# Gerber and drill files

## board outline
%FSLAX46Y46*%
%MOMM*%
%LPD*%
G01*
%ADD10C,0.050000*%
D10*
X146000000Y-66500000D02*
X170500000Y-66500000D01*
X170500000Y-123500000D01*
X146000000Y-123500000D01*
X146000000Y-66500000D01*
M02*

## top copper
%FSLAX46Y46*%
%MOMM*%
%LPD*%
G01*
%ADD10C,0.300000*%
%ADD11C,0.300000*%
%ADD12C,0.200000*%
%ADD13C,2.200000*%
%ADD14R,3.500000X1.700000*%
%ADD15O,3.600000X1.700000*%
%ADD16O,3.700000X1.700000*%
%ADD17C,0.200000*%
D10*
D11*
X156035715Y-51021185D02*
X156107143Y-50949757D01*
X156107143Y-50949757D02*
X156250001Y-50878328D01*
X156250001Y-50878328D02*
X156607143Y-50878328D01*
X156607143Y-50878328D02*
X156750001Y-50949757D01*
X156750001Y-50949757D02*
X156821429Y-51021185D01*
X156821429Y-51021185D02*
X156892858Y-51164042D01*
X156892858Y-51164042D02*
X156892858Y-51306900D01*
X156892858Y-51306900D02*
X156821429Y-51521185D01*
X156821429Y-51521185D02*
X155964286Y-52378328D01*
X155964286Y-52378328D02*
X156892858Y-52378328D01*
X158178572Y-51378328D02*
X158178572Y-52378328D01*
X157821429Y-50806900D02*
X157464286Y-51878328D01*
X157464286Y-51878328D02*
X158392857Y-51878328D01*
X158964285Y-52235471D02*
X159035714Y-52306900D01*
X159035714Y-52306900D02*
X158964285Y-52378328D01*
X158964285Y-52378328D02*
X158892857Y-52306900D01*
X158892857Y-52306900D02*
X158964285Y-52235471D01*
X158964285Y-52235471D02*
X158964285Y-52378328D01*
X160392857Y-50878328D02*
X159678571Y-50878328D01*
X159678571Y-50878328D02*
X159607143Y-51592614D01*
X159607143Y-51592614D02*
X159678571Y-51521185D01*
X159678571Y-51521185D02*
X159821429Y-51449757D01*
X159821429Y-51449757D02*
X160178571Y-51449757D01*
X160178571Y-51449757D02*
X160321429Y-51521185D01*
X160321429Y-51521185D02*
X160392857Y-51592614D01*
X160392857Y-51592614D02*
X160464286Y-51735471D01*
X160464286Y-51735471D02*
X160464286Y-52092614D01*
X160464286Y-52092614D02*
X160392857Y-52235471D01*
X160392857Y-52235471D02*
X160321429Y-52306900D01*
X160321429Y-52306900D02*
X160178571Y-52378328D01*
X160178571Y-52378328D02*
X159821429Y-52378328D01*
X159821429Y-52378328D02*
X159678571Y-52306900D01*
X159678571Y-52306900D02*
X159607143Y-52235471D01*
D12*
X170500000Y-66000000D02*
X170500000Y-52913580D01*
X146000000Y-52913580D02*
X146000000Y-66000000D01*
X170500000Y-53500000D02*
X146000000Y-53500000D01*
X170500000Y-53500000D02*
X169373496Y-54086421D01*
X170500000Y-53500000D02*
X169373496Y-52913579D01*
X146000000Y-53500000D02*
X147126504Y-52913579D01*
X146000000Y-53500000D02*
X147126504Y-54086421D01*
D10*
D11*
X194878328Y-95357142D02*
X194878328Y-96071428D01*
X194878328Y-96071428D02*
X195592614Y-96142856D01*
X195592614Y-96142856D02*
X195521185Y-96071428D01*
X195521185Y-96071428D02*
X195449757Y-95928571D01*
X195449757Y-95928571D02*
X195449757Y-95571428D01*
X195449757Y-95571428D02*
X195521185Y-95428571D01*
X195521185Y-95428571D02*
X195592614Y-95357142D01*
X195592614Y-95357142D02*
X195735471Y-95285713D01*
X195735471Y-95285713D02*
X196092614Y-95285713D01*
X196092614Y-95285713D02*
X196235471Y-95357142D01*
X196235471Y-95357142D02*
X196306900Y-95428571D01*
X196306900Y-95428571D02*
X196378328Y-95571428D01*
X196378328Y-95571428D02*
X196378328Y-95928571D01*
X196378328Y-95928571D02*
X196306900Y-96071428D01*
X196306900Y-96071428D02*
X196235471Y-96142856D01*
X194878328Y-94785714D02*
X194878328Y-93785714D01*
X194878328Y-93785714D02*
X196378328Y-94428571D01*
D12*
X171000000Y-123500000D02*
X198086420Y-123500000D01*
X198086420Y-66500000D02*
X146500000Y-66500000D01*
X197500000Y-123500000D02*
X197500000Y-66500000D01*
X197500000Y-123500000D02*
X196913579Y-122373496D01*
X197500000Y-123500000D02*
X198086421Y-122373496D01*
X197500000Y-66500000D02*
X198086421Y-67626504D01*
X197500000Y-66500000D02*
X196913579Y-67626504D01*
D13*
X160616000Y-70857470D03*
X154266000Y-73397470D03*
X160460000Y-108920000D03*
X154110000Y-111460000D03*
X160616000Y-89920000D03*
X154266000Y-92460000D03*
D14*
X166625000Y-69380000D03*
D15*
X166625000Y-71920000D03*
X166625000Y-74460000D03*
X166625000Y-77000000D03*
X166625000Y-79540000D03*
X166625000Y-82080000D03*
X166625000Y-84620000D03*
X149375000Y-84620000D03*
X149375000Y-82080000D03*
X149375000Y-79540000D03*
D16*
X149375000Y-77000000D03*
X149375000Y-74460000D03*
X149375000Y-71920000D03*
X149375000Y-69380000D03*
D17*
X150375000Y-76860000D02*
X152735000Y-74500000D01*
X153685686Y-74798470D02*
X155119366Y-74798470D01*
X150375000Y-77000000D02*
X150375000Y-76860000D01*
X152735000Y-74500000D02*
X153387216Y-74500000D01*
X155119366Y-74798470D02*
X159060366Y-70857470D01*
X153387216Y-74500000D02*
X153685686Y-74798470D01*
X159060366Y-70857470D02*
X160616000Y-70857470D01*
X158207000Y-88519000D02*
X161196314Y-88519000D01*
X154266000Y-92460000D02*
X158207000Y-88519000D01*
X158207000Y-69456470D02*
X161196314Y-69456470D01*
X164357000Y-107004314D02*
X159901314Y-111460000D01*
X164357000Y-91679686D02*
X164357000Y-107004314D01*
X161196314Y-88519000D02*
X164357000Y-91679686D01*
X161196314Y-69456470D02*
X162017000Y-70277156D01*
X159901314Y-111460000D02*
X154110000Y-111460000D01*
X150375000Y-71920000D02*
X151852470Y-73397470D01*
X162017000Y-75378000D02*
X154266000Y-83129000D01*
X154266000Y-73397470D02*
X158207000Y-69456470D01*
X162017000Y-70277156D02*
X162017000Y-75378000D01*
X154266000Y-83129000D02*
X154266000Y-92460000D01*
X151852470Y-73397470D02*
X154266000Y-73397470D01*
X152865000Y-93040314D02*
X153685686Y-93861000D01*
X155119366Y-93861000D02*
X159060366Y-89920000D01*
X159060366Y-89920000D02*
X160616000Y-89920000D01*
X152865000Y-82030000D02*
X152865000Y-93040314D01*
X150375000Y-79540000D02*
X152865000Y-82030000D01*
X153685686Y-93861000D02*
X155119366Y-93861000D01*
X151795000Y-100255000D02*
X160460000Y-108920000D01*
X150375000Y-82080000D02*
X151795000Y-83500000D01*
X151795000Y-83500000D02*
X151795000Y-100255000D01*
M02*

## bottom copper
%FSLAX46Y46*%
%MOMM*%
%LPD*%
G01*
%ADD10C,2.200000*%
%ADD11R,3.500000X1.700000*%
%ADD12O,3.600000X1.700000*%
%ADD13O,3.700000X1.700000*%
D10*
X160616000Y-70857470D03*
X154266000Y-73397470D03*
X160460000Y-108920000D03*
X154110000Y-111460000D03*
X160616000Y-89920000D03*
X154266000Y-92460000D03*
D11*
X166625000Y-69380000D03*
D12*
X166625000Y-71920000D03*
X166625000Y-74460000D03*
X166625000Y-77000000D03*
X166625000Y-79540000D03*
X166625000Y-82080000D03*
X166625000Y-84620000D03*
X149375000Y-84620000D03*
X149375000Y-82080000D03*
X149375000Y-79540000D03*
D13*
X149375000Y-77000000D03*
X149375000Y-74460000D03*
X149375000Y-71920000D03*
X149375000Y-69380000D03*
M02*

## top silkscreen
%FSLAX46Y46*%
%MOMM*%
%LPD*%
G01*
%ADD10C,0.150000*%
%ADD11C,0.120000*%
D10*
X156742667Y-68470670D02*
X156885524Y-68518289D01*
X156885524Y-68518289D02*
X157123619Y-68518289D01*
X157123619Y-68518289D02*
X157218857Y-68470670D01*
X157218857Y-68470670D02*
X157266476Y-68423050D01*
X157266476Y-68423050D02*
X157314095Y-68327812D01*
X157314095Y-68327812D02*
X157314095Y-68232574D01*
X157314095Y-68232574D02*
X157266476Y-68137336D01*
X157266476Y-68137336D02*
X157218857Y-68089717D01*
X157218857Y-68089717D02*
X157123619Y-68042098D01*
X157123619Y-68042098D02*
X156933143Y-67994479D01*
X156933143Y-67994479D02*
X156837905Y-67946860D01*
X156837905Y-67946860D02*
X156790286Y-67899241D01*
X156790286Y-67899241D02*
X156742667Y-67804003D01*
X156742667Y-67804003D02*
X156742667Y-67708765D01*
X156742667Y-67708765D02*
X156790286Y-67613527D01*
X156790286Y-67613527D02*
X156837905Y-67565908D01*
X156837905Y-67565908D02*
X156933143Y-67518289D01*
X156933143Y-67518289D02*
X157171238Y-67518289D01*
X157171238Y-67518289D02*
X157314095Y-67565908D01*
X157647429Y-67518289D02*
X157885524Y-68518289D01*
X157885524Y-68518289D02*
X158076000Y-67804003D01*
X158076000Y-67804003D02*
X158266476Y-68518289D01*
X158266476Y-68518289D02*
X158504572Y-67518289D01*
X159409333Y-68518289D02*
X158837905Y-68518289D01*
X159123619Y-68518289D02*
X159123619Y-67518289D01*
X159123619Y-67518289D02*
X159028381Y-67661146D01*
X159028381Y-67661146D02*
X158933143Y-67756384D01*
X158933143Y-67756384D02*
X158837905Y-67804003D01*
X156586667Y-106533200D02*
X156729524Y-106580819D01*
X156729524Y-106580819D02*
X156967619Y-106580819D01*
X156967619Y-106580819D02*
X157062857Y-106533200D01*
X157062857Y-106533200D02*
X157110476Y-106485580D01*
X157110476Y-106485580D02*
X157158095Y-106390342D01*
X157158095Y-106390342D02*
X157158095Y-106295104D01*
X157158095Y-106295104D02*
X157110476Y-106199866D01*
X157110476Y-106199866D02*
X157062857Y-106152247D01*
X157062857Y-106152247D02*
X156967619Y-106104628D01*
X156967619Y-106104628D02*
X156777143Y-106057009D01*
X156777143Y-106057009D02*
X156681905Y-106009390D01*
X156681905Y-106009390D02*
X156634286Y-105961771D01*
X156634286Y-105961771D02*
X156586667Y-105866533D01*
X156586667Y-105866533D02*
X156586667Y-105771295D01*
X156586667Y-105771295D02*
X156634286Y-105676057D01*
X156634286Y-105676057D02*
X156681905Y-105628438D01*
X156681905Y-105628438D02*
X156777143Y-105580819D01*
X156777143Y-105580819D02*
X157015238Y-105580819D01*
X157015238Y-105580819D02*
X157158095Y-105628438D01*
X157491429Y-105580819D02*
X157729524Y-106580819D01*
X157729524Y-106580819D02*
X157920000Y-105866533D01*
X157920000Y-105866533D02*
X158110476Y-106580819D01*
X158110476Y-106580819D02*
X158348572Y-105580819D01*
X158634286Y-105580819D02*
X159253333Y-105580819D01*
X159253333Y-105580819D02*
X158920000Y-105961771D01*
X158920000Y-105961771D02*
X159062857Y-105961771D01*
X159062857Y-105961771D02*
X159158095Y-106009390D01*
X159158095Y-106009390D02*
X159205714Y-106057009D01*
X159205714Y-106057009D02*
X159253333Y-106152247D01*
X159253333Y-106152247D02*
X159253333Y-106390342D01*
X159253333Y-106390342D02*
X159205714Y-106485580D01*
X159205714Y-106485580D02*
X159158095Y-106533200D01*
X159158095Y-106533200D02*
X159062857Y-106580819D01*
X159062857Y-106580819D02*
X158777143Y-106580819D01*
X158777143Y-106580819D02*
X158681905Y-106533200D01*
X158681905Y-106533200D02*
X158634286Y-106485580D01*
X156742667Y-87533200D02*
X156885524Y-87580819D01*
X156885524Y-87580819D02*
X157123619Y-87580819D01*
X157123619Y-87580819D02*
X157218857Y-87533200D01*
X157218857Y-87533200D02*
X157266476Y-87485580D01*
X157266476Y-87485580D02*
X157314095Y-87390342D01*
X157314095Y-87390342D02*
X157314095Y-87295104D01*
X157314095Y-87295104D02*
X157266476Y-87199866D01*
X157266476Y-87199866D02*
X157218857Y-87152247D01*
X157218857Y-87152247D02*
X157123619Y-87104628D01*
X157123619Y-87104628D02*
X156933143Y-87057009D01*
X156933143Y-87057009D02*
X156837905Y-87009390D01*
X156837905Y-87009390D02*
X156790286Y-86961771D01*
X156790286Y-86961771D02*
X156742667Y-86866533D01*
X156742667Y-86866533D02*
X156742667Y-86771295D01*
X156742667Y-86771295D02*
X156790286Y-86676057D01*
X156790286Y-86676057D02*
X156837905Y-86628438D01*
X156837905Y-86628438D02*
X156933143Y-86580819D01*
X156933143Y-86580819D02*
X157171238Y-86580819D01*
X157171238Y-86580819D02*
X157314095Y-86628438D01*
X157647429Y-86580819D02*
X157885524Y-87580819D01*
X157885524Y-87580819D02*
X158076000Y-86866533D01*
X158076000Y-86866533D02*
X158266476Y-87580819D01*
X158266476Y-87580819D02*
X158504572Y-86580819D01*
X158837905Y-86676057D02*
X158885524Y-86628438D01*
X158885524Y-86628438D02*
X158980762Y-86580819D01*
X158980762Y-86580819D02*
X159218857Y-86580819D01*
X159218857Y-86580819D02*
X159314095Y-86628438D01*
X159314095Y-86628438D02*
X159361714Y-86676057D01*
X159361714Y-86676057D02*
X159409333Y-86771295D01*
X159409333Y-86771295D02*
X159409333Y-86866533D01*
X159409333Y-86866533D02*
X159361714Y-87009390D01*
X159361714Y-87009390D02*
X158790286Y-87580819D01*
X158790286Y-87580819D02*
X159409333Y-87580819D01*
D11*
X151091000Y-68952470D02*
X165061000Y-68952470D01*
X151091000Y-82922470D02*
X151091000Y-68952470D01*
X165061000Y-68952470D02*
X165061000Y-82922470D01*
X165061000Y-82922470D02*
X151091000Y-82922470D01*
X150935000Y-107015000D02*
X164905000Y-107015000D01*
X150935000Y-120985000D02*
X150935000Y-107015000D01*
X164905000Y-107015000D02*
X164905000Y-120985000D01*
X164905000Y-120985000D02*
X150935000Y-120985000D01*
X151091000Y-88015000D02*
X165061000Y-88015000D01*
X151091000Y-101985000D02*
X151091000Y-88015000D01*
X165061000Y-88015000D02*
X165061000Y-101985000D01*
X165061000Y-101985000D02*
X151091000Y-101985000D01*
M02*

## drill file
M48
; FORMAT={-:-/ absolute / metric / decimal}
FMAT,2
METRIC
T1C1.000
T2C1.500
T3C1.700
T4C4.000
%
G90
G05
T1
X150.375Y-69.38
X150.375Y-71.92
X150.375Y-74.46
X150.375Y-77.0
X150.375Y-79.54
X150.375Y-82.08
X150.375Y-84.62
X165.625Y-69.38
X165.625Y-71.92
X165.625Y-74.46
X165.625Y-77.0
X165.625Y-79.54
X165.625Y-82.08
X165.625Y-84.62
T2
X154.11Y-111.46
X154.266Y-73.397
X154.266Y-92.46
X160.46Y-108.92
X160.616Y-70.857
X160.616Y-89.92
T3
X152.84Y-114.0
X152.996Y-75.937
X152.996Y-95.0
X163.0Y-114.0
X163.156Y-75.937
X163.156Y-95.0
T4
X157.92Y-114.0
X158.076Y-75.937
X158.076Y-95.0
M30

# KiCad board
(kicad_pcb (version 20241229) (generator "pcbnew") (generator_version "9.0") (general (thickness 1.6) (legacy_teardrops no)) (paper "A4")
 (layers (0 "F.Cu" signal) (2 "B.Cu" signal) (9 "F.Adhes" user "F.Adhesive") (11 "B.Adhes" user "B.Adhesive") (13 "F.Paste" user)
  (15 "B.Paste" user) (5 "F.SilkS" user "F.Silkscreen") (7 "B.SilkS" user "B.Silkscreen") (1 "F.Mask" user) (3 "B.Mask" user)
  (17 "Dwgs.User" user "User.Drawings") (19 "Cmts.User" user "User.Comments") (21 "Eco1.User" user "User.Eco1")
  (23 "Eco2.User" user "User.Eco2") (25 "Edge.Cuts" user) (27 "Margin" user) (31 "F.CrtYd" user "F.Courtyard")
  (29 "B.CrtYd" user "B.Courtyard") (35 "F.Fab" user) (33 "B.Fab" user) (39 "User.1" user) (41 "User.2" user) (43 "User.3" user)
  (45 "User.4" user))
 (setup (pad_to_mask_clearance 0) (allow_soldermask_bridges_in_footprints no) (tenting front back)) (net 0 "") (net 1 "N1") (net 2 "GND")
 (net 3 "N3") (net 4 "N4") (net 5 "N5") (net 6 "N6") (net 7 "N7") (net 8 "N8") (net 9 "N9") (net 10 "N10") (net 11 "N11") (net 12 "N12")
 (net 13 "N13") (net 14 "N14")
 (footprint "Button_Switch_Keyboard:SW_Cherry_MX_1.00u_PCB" (layer "F.Cu") (at 160.616 70.85747)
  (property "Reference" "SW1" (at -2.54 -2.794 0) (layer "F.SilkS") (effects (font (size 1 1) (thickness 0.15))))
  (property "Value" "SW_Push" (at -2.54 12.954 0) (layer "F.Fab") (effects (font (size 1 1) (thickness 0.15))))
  (fp_line (start -9.525 -1.905) (end 4.445 -1.905) (stroke (width 0.12) (type solid)) (layer "F.SilkS"))
  (fp_line (start -9.525 12.065) (end -9.525 -1.905) (stroke (width 0.12) (type solid)) (layer "F.SilkS"))
  (fp_line (start 4.445 -1.905) (end 4.445 12.065) (stroke (width 0.12) (type solid)) (layer "F.SilkS"))
  (fp_line (start 4.445 12.065) (end -9.525 12.065) (stroke (width 0.12) (type solid)) (layer "F.SilkS"))
  (pad "" np_thru_hole circle (at -7.62 5.08) (size 1.7 1.7) (drill 1.7) (layers "*.Cu" "*.Mask"))
  (pad "" np_thru_hole circle (at -2.54 5.08) (size 4 4) (drill 4) (layers "*.Cu" "*.Mask"))
  (pad "" np_thru_hole circle (at 2.54 5.08) (size 1.7 1.7) (drill 1.7) (layers "*.Cu" "*.Mask"))
  (pad "1" thru_hole circle (at 0 0) (size 2.2 2.2) (drill 1.5) (layers "*.Cu" "*.Mask") (remove_unused_layers no) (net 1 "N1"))
  (pad "2" thru_hole circle (at -6.35 2.54) (size 2.2 2.2) (drill 1.5) (layers "*.Cu" "*.Mask") (remove_unused_layers no) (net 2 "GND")))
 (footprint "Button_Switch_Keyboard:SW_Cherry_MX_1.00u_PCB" (layer "F.Cu") (at 160.46 108.92)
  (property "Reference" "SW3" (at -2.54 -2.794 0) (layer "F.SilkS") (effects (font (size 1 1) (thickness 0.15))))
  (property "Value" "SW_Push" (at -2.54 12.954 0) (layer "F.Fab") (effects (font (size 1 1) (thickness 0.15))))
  (fp_line (start -9.525 -1.905) (end 4.445 -1.905) (stroke (width 0.12) (type solid)) (layer "F.SilkS"))
  (fp_line (start -9.525 12.065) (end -9.525 -1.905) (stroke (width 0.12) (type solid)) (layer "F.SilkS"))
  (fp_line (start 4.445 -1.905) (end 4.445 12.065) (stroke (width 0.12) (type solid)) (layer "F.SilkS"))
  (fp_line (start 4.445 12.065) (end -9.525 12.065) (stroke (width 0.12) (type solid)) (layer "F.SilkS"))
  (pad "" np_thru_hole circle (at -7.62 5.08) (size 1.7 1.7) (drill 1.7) (layers "*.Cu" "*.Mask"))
  (pad "" np_thru_hole circle (at -2.54 5.08) (size 4 4) (drill 4) (layers "*.Cu" "*.Mask"))
  (pad "" np_thru_hole circle (at 2.54 5.08) (size 1.7 1.7) (drill 1.7) (layers "*.Cu" "*.Mask"))
  (pad "1" thru_hole circle (at 0 0) (size 2.2 2.2) (drill 1.5) (layers "*.Cu" "*.Mask") (remove_unused_layers no) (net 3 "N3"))
  (pad "2" thru_hole circle (at -6.35 2.54) (size 2.2 2.2) (drill 1.5) (layers "*.Cu" "*.Mask") (remove_unused_layers no) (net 2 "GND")))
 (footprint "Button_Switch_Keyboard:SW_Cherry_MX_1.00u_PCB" (layer "F.Cu") (at 160.616 89.92)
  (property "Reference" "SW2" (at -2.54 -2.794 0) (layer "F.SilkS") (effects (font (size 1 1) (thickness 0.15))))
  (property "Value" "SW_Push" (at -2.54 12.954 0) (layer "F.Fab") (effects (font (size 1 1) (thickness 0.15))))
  (fp_line (start -9.525 -1.905) (end 4.445 -1.905) (stroke (width 0.12) (type solid)) (layer "F.SilkS"))
  (fp_line (start -9.525 12.065) (end -9.525 -1.905) (stroke (width 0.12) (type solid)) (layer "F.SilkS"))
  (fp_line (start 4.445 -1.905) (end 4.445 12.065) (stroke (width 0.12) (type solid)) (layer "F.SilkS"))
  (fp_line (start 4.445 12.065) (end -9.525 12.065) (stroke (width 0.12) (type solid)) (layer "F.SilkS"))
  (pad "" np_thru_hole circle (at -7.62 5.08) (size 1.7 1.7) (drill 1.7) (layers "*.Cu" "*.Mask"))
  (pad "" np_thru_hole circle (at -2.54 5.08) (size 4 4) (drill 4) (layers "*.Cu" "*.Mask"))
  (pad "" np_thru_hole circle (at 2.54 5.08) (size 1.7 1.7) (drill 1.7) (layers "*.Cu" "*.Mask"))
  (pad "1" thru_hole circle (at 0 0) (size 2.2 2.2) (drill 1.5) (layers "*.Cu" "*.Mask") (remove_unused_layers no) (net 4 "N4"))
  (pad "2" thru_hole circle (at -6.35 2.54) (size 2.2 2.2) (drill 1.5) (layers "*.Cu" "*.Mask") (remove_unused_layers no) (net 2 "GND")))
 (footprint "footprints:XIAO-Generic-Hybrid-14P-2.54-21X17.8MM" (layer "B.Cu") (at 158 77 180)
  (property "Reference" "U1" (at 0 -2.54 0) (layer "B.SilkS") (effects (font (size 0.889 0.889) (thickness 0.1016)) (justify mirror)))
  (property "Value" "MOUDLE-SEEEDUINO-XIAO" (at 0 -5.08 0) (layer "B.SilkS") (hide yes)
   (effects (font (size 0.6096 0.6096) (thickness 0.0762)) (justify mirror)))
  (pad "1" thru_hole rect (at -7.625 7.62 180) (size 3.5 1.7) (drill 1 (offset -1 0)) (layers "*.Cu" "*.Mask") (remove_unused_layers no)
   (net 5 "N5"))
  (pad "2" thru_hole oval (at -7.625 5.08 180) (size 3.6 1.7) (drill 1 (offset -1 0)) (layers "*.Cu" "*.Mask") (remove_unused_layers no)
   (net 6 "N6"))
  (pad "3" thru_hole oval (at -7.625 2.54 180) (size 3.6 1.7) (drill 1 (offset -1 0)) (layers "*.Cu" "*.Mask") (remove_unused_layers no)
   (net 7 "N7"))
  (pad "4" thru_hole oval (at -7.625 0 180) (size 3.6 1.7) (drill 1 (offset -1 0)) (layers "*.Cu" "*.Mask") (remove_unused_layers no)
   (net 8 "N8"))
  (pad "5" thru_hole oval (at -7.625 -2.54 180) (size 3.6 1.7) (drill 1 (offset -1 0)) (layers "*.Cu" "*.Mask") (remove_unused_layers no)
   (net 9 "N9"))
  (pad "6" thru_hole oval (at -7.625 -5.08) (size 3.6 1.7) (drill 1 (offset 1 0)) (layers "*.Cu" "*.Mask") (remove_unused_layers no)
   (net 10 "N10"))
  (pad "7" thru_hole oval (at -7.625 -7.62 180) (size 3.6 1.7) (drill 1 (offset -1 0)) (layers "*.Cu" "*.Mask") (remove_unused_layers no)
   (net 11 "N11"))
  (pad "8" thru_hole oval (at 7.625 -7.62 180) (size 3.6 1.7) (drill 1 (offset 1 0)) (layers "*.Cu" "*.Mask") (remove_unused_layers no)
   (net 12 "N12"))
  (pad "9" thru_hole oval (at 7.625 -5.08 180) (size 3.6 1.7) (drill 1 (offset 1 0)) (layers "*.Cu" "*.Mask") (remove_unused_layers no)
   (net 3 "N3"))
  (pad "10" thru_hole oval (at 7.625 -2.54 180) (size 3.6 1.7) (drill 1 (offset 1 0)) (layers "*.Cu" "*.Mask") (remove_unused_layers no)
   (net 4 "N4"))
  (pad "11" thru_hole oval (at 7.625 0 180) (size 3.7 1.7) (drill 1 (offset 1 0)) (layers "*.Cu" "*.Mask") (remove_unused_layers no)
   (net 1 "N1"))
  (pad "12" thru_hole oval (at 7.625 2.54 180) (size 3.7 1.7) (drill 1 (offset 1 0)) (layers "*.Cu" "*.Mask") (remove_unused_layers no)
   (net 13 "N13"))
  (pad "13" thru_hole oval (at 7.625 5.08 180) (size 3.7 1.7) (drill 1 (offset 1 0)) (layers "*.Cu" "*.Mask") (remove_unused_layers no)
   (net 2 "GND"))
  (pad "14" thru_hole oval (at 7.625 7.62 180) (size 3.7 1.7) (drill 1 (offset 1 0)) (layers "*.Cu" "*.Mask") (remove_unused_layers no)
   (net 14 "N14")))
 (gr_rect (start 146 66.5) (end 170.5 123.5) (stroke (width 0.05) (type default)) (fill no) (layer "Edge.Cuts"))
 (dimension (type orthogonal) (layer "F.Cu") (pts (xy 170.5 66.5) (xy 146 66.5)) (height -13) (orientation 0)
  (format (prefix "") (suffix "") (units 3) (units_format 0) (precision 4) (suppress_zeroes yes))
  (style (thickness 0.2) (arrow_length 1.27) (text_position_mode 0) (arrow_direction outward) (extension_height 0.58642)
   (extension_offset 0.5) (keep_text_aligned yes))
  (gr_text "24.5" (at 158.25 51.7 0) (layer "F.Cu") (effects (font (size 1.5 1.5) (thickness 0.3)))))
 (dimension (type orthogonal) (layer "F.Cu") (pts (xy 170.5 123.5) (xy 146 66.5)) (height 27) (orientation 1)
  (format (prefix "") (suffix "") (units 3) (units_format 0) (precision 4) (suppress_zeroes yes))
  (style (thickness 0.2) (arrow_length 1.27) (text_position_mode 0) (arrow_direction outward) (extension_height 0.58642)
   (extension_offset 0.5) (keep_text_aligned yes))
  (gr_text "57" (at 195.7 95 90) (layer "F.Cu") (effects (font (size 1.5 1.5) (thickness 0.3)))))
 (segment (start 150.375 76.86) (end 152.735 74.5) (width 0.2) (layer "F.Cu") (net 1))
 (segment (start 153.685686 74.79847) (end 155.119366 74.79847) (width 0.2) (layer "F.Cu") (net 1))
 (segment (start 150.375 77) (end 150.375 76.86) (width 0.2) (layer "F.Cu") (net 1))
 (segment (start 152.735 74.5) (end 153.387216 74.5) (width 0.2) (layer "F.Cu") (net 1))
 (segment (start 155.119366 74.79847) (end 159.060366 70.85747) (width 0.2) (layer "F.Cu") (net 1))
 (segment (start 153.387216 74.5) (end 153.685686 74.79847) (width 0.2) (layer "F.Cu") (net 1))
 (segment (start 159.060366 70.85747) (end 160.616 70.85747) (width 0.2) (layer "F.Cu") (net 1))
 (segment (start 158.207 88.519) (end 161.196314 88.519) (width 0.2) (layer "F.Cu") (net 2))
 (segment (start 154.266 92.46) (end 158.207 88.519) (width 0.2) (layer "F.Cu") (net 2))
 (segment (start 158.207 69.45647) (end 161.196314 69.45647) (width 0.2) (layer "F.Cu") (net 2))
 (segment (start 164.357 107.004314) (end 159.901314 111.46) (width 0.2) (layer "F.Cu") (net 2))
 (segment (start 164.357 91.679686) (end 164.357 107.004314) (width 0.2) (layer "F.Cu") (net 2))
 (segment (start 161.196314 88.519) (end 164.357 91.679686) (width 0.2) (layer "F.Cu") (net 2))
 (segment (start 161.196314 69.45647) (end 162.017 70.277156) (width 0.2) (layer "F.Cu") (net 2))
 (segment (start 159.901314 111.46) (end 154.11 111.46) (width 0.2) (layer "F.Cu") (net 2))
 (segment (start 150.375 71.92) (end 151.85247 73.39747) (width 0.2) (layer "F.Cu") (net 2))
 (segment (start 162.017 75.378) (end 154.266 83.129) (width 0.2) (layer "F.Cu") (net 2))
 (segment (start 154.266 73.39747) (end 158.207 69.45647) (width 0.2) (layer "F.Cu") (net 2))
 (segment (start 162.017 70.277156) (end 162.017 75.378) (width 0.2) (layer "F.Cu") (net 2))
 (segment (start 154.266 83.129) (end 154.266 92.46) (width 0.2) (layer "F.Cu") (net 2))
 (segment (start 151.85247 73.39747) (end 154.266 73.39747) (width 0.2) (layer "F.Cu") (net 2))
 (segment (start 152.865 93.040314) (end 153.685686 93.861) (width 0.2) (layer "F.Cu") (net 4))
 (segment (start 155.119366 93.861) (end 159.060366 89.92) (width 0.2) (layer "F.Cu") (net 4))
 (segment (start 159.060366 89.92) (end 160.616 89.92) (width 0.2) (layer "F.Cu") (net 4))
 (segment (start 152.865 82.03) (end 152.865 93.040314) (width 0.2) (layer "F.Cu") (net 4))
 (segment (start 150.375 79.54) (end 152.865 82.03) (width 0.2) (layer "F.Cu") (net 4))
 (segment (start 153.685686 93.861) (end 155.119366 93.861) (width 0.2) (layer "F.Cu") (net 4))
 (segment (start 151.795 100.255) (end 160.46 108.92) (width 0.2) (layer "F.Cu") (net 3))
 (segment (start 150.375 82.08) (end 151.795 83.5) (width 0.2) (layer "F.Cu") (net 3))
 (segment (start 151.795 83.5) (end 151.795 100.255) (width 0.2) (layer "F.Cu") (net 3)))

